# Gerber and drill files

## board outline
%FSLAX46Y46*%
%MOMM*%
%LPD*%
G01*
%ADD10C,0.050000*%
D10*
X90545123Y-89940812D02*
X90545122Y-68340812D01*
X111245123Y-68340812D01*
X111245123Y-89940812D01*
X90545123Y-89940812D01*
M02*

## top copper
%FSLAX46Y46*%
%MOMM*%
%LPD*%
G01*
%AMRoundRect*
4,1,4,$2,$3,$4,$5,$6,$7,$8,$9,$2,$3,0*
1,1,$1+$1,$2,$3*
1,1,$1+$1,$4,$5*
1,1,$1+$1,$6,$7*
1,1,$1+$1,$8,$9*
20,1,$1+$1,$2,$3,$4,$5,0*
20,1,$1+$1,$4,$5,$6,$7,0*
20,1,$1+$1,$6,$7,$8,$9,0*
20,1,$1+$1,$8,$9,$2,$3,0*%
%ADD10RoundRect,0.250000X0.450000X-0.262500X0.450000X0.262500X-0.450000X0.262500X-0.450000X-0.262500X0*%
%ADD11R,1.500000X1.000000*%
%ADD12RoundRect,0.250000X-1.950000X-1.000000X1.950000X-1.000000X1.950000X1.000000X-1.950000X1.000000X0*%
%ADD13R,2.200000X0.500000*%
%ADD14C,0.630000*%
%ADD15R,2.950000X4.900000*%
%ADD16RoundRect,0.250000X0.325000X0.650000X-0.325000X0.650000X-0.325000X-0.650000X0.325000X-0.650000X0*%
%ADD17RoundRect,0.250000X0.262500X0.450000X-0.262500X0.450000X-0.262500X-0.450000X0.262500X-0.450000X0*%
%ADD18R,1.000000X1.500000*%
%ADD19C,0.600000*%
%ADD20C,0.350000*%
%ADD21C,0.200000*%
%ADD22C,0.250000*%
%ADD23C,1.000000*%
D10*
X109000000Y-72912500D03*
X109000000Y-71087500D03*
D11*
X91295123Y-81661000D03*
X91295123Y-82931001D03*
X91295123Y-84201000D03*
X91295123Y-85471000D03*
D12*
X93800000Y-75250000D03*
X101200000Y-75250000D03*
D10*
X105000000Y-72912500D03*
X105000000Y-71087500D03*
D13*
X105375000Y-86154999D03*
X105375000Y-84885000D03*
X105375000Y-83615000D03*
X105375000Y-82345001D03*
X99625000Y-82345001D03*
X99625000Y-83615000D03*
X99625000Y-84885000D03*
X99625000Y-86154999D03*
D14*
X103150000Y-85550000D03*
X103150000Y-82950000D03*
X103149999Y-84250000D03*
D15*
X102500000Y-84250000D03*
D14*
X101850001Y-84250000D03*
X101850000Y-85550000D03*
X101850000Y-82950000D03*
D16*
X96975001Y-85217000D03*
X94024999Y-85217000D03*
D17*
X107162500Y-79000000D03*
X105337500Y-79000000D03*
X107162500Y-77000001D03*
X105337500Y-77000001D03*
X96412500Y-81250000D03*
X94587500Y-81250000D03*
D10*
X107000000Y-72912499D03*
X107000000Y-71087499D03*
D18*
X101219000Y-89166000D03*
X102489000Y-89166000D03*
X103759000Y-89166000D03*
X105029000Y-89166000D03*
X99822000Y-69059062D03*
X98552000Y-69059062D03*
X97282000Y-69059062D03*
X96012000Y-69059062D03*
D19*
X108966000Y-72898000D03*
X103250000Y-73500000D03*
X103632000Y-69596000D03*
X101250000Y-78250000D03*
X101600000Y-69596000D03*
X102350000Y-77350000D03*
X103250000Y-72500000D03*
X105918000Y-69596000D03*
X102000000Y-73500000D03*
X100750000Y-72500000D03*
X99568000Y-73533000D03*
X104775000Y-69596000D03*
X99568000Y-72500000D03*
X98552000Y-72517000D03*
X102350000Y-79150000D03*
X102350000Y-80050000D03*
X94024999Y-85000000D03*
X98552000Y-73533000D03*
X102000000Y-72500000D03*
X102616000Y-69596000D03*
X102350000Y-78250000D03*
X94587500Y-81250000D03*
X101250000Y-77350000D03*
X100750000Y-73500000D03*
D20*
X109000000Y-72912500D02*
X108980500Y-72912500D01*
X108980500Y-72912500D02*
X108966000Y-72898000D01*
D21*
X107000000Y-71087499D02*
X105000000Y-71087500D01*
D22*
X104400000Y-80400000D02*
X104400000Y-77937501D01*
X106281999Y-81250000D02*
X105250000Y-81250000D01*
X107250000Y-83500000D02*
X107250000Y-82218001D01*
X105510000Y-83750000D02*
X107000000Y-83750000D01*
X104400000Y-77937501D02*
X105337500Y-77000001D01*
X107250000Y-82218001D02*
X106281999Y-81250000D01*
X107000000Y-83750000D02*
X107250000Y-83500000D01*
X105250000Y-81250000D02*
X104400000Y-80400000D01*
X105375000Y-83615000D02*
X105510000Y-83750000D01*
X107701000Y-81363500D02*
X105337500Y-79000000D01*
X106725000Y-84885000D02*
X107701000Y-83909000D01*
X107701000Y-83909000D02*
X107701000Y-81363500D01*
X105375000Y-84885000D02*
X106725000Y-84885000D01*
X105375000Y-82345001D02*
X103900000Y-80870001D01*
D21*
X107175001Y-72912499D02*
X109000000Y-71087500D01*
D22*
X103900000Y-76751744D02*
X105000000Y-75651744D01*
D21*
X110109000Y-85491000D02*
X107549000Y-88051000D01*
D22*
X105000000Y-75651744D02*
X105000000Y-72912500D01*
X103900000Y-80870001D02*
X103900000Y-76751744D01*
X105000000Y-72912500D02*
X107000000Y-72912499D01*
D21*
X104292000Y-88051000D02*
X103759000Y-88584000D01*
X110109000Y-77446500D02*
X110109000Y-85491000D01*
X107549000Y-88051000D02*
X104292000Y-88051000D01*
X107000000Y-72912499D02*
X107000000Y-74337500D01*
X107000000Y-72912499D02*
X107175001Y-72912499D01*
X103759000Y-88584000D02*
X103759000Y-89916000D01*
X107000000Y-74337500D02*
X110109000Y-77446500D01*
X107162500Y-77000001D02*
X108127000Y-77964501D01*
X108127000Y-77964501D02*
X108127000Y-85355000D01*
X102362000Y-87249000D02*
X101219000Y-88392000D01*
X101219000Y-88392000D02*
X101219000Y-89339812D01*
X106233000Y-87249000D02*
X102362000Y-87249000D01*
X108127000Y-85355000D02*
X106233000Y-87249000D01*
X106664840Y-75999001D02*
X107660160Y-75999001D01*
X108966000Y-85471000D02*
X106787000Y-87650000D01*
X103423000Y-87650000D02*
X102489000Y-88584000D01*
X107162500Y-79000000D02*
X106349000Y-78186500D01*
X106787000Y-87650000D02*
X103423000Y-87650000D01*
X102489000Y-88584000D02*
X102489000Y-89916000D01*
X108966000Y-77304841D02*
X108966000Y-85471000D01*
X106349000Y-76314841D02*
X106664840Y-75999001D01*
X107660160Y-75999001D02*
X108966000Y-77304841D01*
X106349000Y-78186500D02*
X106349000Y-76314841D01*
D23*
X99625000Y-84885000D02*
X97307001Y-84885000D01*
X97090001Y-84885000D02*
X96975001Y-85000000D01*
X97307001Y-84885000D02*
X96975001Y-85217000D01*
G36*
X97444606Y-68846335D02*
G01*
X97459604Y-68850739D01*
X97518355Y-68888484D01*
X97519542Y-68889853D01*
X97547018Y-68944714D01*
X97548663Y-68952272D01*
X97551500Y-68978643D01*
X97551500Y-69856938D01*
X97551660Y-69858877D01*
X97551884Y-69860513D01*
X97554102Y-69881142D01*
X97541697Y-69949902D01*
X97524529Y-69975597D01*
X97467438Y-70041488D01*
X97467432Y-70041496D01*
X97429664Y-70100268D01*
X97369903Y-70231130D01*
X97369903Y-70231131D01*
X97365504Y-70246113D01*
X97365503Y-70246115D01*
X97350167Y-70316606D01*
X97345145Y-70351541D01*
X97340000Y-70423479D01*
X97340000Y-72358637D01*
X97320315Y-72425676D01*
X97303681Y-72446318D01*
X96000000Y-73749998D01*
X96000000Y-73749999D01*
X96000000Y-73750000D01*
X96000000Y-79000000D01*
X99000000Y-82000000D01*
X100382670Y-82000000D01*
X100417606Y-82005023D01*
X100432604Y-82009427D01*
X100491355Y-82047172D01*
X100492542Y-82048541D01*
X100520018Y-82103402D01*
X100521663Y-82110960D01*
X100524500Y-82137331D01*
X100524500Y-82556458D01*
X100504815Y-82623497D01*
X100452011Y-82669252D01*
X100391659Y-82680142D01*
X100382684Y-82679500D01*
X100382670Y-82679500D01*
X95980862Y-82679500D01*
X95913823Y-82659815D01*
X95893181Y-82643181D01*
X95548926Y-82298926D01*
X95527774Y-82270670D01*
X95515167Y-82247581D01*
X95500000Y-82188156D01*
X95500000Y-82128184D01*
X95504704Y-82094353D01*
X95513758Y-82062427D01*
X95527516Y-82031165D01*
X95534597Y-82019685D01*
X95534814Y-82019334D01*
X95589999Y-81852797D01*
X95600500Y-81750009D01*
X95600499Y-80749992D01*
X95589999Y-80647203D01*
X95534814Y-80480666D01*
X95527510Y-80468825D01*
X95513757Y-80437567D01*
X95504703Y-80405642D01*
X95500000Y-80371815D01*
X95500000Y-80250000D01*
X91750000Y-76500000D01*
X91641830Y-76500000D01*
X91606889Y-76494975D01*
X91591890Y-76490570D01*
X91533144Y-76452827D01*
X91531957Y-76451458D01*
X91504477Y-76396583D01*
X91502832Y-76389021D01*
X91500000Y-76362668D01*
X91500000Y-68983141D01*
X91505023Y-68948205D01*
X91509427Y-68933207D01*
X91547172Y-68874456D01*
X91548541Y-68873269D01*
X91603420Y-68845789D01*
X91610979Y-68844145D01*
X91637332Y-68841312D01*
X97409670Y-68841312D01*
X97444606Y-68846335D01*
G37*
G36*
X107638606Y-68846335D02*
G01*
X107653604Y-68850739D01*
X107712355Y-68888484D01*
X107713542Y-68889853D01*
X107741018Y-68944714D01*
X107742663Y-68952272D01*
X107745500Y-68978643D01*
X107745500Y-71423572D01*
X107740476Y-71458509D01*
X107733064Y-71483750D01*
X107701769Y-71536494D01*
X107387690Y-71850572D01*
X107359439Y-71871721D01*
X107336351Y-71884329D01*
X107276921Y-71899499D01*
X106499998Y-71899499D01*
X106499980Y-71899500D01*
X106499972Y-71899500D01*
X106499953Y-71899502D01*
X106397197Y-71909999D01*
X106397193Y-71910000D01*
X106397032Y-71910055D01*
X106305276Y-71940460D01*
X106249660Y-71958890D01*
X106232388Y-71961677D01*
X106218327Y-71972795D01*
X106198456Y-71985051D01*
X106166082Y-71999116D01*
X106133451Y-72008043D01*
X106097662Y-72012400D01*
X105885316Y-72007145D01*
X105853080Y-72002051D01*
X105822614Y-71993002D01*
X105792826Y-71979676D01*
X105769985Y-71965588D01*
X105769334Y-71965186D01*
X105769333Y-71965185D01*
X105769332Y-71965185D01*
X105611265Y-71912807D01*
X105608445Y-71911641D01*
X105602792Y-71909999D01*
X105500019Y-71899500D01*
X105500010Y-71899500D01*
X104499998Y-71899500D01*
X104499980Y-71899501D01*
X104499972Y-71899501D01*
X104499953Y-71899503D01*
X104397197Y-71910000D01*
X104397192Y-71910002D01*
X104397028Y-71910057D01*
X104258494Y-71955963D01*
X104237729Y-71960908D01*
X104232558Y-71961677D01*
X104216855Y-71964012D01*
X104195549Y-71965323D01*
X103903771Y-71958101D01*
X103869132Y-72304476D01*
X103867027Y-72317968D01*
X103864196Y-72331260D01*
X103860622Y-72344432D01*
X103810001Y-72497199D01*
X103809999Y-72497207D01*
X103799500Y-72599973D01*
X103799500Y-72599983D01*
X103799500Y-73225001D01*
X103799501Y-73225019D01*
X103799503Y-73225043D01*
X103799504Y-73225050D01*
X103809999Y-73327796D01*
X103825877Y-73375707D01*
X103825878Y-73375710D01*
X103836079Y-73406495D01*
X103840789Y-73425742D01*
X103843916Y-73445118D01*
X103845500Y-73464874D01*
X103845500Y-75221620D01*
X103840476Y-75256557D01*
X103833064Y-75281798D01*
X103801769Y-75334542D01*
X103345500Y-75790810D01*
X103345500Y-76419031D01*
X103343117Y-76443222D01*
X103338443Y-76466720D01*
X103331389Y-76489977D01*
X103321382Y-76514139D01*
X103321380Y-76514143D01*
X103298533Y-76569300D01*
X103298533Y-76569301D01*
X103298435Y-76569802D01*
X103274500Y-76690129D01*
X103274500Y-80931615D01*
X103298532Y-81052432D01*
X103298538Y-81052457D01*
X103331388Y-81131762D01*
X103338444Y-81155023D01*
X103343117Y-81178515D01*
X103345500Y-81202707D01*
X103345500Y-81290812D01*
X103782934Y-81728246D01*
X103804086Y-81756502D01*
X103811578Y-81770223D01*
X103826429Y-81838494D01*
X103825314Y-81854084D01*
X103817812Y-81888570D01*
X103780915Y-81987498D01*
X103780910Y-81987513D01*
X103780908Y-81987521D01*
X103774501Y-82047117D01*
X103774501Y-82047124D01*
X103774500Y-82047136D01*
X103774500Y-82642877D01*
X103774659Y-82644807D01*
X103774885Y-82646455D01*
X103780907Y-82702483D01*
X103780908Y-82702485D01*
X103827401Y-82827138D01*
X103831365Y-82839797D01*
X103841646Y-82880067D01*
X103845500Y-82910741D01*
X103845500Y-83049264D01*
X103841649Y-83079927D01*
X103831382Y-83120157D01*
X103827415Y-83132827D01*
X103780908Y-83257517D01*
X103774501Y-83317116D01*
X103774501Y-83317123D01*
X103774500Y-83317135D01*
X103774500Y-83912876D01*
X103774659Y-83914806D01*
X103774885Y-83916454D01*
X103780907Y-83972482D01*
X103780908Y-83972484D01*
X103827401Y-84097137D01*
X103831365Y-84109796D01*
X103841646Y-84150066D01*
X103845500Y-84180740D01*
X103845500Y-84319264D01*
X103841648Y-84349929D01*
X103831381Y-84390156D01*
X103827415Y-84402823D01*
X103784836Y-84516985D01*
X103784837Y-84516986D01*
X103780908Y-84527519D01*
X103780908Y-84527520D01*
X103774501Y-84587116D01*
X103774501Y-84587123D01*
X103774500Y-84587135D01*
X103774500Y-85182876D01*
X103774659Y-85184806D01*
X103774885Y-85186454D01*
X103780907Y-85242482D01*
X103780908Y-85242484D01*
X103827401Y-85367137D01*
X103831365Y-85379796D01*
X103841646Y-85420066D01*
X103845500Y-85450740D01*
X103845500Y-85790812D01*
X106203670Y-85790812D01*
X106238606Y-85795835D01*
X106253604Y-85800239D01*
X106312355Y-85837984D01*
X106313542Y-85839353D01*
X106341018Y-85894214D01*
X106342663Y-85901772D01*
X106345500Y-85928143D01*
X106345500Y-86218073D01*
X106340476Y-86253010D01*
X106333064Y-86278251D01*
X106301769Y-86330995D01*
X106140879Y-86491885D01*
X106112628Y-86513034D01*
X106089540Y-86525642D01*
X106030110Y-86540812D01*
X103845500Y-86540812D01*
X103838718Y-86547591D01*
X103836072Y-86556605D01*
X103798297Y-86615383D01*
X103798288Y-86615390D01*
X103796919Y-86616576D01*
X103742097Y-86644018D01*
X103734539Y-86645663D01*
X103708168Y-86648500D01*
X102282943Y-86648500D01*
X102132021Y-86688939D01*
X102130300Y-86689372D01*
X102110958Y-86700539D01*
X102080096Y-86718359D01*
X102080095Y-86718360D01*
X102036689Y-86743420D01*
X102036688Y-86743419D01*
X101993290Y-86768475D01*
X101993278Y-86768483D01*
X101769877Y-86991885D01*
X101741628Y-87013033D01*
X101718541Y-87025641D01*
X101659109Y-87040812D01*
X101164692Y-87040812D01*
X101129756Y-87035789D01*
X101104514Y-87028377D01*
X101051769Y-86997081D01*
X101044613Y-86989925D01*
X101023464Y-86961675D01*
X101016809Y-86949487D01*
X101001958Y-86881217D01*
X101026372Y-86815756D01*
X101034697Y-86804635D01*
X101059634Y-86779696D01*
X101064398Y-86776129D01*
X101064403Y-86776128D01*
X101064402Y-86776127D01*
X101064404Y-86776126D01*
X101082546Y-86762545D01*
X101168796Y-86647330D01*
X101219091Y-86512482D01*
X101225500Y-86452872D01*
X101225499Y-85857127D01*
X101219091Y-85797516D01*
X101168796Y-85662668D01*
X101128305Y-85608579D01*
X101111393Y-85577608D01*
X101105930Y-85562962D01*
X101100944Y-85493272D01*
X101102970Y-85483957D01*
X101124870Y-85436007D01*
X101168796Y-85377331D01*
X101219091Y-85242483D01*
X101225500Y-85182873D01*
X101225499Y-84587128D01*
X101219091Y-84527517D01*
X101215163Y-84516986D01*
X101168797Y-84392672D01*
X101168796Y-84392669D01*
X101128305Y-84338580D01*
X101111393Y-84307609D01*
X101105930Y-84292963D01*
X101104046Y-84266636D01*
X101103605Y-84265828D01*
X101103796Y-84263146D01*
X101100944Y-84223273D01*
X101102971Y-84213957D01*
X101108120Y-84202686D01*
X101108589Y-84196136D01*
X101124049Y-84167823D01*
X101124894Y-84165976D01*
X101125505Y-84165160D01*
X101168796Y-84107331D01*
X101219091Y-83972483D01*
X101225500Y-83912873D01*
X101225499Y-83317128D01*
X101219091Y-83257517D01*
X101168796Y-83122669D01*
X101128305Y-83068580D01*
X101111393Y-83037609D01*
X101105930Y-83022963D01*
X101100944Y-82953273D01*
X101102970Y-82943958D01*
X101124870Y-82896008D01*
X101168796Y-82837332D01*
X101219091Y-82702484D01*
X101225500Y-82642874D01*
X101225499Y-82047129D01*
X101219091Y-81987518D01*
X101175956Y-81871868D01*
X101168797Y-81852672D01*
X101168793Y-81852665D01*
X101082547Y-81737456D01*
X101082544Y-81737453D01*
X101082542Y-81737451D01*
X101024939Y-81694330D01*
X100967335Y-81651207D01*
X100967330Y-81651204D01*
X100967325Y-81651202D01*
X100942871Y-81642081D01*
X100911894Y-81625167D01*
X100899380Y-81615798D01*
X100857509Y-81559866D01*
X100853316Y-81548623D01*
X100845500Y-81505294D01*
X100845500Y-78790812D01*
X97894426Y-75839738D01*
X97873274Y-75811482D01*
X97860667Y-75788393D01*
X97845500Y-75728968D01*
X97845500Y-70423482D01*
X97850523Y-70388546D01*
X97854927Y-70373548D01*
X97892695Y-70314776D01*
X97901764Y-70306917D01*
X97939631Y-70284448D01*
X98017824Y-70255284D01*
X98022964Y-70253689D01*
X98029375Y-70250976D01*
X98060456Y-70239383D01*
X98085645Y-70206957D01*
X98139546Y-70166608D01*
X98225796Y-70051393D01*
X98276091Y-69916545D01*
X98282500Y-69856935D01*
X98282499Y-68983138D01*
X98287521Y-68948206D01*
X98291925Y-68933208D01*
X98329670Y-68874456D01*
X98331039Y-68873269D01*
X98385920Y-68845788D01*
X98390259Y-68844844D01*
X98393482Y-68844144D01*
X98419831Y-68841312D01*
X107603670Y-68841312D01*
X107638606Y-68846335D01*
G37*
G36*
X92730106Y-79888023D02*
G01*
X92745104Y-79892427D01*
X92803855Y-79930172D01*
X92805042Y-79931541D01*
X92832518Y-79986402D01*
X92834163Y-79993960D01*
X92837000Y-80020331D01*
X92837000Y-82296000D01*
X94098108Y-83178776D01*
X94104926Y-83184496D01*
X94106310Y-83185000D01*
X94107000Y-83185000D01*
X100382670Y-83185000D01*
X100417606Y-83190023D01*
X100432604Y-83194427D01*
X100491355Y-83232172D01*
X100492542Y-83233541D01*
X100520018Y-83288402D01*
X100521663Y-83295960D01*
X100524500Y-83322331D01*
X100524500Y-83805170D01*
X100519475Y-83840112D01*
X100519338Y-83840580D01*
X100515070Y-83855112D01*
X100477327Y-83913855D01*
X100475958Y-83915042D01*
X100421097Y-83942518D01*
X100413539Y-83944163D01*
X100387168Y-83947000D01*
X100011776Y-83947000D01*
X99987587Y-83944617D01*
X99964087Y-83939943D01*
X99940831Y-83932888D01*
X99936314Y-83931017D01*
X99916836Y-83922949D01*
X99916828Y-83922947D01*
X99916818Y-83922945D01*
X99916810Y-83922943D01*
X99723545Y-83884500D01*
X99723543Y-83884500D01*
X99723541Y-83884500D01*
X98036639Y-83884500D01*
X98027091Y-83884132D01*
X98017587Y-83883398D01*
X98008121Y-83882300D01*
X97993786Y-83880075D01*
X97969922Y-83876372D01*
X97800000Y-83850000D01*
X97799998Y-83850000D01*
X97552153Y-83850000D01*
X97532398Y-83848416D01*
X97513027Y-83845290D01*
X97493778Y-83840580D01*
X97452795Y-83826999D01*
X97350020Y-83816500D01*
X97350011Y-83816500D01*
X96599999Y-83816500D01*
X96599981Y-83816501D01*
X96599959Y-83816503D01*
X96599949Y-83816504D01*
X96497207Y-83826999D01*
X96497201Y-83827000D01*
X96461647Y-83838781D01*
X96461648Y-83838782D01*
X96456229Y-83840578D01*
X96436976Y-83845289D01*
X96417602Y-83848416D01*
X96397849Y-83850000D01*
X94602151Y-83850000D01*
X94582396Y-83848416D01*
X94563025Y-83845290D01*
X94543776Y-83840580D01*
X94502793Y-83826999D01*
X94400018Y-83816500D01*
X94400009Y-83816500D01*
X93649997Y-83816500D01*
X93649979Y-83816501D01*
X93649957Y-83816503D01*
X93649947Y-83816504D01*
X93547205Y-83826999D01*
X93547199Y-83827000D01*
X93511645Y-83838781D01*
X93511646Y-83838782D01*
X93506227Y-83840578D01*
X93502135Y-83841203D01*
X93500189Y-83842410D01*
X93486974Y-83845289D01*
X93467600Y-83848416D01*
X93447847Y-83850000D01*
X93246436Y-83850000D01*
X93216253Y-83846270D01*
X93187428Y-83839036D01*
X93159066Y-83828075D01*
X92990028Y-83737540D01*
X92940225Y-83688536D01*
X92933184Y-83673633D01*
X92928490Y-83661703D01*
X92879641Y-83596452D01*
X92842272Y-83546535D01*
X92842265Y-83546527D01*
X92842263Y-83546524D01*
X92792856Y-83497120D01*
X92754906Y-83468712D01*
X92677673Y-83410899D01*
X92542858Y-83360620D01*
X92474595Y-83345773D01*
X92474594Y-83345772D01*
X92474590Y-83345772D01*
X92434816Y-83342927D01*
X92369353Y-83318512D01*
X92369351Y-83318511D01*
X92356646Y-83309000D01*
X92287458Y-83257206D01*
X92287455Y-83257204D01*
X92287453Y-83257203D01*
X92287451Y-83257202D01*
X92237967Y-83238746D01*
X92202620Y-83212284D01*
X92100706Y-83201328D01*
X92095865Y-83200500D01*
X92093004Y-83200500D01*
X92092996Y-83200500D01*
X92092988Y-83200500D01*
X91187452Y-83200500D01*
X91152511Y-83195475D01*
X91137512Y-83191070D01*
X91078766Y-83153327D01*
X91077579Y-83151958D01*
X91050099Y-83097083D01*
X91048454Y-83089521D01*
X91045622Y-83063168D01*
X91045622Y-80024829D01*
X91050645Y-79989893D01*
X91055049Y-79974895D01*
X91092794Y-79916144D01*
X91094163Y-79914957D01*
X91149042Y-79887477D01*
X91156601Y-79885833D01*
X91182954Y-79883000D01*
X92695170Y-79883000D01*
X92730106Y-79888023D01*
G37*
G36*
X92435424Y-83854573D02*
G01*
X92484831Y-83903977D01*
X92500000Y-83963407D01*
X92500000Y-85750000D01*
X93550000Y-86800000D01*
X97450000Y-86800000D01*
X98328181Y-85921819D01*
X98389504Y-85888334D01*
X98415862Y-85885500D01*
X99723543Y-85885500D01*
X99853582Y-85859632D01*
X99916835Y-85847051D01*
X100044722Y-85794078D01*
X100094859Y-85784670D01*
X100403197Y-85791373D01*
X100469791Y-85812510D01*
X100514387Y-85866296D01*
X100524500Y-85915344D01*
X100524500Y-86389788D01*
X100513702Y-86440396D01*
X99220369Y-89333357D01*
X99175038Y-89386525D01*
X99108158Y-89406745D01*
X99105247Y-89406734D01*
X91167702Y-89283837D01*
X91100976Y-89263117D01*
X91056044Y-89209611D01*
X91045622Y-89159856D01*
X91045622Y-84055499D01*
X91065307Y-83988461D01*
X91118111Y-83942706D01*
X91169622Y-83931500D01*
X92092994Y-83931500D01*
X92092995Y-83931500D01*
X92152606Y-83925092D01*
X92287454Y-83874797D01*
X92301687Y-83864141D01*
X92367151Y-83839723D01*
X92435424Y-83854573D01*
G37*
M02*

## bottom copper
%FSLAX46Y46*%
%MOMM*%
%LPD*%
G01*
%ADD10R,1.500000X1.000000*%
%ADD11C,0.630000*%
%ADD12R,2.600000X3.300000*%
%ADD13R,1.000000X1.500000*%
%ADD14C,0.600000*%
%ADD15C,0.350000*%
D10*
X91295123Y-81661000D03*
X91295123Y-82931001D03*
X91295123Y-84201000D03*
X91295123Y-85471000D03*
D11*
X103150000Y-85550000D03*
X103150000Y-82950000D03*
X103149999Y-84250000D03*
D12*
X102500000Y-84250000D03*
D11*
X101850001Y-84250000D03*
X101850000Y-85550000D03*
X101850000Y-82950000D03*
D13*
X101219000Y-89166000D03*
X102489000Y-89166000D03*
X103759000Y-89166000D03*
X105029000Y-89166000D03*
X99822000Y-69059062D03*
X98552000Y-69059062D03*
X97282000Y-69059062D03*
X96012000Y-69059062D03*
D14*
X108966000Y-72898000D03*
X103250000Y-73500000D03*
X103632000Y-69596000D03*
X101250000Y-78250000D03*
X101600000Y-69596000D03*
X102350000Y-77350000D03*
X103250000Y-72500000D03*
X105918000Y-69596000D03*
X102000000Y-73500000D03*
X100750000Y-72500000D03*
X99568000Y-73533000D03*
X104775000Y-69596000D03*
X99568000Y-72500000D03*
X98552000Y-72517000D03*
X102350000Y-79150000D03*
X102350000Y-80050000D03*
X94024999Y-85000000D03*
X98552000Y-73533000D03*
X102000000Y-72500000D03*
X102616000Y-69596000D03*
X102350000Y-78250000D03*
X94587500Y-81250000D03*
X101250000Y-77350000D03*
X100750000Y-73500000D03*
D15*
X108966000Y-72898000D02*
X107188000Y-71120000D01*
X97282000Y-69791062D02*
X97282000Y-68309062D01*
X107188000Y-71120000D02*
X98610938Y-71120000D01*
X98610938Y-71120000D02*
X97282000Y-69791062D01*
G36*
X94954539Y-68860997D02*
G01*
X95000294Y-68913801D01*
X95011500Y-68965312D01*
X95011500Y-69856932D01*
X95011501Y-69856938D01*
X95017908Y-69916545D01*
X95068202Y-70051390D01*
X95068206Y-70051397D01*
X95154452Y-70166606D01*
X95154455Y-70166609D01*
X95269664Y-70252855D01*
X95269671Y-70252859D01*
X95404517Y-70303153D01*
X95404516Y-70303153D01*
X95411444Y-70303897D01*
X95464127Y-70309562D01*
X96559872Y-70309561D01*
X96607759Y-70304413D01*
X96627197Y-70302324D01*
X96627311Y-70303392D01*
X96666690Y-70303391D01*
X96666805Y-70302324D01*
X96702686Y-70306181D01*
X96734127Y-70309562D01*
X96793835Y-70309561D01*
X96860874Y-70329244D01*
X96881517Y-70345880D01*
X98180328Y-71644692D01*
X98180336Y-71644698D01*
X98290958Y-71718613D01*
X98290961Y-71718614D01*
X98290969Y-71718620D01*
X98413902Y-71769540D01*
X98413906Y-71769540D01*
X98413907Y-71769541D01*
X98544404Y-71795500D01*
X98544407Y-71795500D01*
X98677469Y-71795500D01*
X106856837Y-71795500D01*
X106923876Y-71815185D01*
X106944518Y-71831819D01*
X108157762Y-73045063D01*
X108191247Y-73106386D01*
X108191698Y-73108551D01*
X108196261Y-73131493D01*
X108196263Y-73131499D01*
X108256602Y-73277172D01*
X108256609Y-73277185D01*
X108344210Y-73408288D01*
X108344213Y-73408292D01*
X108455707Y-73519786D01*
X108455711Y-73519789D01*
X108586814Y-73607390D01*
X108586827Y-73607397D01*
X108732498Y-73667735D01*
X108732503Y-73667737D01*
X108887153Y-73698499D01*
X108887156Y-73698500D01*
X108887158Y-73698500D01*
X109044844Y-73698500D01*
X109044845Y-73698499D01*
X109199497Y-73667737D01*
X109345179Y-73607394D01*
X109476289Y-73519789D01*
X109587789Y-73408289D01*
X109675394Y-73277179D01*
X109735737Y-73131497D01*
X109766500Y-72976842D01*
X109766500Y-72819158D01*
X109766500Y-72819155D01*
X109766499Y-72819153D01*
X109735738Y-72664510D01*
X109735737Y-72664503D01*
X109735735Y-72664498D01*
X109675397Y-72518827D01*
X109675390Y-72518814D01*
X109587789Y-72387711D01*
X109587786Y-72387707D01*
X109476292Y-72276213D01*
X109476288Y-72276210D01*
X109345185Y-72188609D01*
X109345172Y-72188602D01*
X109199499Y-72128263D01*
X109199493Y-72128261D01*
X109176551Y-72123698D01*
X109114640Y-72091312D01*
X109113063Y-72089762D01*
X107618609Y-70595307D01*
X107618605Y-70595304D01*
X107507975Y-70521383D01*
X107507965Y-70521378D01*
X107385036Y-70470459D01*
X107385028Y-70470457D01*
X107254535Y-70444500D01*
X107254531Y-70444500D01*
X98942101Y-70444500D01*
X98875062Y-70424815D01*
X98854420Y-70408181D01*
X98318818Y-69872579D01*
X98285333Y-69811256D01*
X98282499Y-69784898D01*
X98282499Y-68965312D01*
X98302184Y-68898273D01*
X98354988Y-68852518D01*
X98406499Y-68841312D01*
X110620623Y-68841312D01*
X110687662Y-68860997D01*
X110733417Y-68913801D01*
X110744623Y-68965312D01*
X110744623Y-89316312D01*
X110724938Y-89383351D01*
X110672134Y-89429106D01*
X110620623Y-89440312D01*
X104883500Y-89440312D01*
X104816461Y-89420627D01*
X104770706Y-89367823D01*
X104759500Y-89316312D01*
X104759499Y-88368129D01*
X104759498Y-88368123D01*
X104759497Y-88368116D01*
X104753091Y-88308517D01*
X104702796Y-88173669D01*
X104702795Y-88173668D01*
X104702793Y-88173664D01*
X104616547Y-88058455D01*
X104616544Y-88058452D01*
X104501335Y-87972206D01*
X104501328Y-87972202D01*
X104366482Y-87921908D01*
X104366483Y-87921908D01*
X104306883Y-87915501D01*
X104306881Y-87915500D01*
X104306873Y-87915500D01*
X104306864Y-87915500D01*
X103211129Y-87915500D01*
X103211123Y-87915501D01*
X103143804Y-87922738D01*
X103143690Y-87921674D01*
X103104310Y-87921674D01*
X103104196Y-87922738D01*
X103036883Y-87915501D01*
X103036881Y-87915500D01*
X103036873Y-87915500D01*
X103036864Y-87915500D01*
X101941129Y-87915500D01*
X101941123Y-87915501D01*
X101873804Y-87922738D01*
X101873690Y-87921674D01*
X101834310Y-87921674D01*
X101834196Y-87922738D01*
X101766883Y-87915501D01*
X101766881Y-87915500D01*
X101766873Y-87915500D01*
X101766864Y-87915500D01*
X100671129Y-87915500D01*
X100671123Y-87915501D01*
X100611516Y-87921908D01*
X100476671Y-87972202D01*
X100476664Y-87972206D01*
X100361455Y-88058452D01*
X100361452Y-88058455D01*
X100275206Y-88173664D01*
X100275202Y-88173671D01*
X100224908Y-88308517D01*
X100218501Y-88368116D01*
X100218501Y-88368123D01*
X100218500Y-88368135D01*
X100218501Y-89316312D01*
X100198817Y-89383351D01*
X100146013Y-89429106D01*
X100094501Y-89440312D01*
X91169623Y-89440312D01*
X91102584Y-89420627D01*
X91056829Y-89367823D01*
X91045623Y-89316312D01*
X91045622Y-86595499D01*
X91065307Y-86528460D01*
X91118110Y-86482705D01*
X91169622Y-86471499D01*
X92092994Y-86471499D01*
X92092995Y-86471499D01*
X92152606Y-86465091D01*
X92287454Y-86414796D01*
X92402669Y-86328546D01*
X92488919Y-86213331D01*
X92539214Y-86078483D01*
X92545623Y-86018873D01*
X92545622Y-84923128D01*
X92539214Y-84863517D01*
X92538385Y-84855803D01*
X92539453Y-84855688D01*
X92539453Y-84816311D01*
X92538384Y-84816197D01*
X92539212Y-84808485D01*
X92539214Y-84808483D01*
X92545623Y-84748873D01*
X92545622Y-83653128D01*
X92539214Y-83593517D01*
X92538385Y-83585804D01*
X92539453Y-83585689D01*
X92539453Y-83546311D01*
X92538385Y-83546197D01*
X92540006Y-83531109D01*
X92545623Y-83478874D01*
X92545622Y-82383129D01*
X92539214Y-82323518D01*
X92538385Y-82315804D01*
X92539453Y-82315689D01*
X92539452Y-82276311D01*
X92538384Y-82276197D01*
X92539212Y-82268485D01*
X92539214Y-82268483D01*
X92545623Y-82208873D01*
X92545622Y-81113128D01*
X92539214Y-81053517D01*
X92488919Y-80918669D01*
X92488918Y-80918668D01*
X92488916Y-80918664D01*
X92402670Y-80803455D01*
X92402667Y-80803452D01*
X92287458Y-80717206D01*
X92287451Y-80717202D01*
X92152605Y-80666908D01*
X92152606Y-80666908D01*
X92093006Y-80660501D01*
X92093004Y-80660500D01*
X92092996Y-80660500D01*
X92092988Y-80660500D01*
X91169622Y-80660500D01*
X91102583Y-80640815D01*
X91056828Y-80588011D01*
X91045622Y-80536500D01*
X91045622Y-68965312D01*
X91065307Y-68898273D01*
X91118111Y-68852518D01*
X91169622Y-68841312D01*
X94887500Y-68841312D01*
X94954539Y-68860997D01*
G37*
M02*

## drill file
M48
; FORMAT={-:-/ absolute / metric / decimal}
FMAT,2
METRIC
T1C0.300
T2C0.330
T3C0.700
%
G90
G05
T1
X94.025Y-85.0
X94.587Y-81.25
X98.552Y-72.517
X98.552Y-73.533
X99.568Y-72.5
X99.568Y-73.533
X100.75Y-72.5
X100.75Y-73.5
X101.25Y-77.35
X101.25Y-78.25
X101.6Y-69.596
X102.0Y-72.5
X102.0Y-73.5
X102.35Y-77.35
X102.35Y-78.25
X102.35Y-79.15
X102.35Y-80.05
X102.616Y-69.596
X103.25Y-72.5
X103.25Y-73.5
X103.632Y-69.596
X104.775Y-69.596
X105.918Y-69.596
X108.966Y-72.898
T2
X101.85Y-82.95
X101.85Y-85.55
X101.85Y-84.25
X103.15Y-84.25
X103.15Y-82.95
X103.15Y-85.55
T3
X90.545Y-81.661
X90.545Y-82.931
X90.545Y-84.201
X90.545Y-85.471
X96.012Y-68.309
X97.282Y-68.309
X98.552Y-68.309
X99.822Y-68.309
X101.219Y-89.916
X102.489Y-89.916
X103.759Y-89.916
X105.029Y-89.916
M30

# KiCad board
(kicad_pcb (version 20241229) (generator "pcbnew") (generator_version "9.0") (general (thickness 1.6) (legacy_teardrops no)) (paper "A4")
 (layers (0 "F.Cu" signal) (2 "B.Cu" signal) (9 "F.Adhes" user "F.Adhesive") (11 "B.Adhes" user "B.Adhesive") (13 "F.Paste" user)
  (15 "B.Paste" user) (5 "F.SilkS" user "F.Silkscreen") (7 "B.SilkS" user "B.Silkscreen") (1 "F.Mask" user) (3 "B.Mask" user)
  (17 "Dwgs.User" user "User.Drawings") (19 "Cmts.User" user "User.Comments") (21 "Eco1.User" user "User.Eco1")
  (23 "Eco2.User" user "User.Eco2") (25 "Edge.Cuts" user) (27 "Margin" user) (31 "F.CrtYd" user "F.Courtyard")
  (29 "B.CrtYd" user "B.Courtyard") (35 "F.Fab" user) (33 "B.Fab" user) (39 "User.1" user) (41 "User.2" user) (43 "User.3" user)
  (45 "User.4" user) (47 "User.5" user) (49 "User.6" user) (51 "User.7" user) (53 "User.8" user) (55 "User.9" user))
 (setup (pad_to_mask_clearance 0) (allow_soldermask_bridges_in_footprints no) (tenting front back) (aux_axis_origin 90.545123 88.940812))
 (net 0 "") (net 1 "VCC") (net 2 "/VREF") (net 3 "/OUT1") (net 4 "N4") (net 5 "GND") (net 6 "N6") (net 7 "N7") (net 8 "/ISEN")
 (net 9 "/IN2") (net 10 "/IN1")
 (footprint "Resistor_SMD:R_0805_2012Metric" (layer "F.Cu") (at 109 72 90)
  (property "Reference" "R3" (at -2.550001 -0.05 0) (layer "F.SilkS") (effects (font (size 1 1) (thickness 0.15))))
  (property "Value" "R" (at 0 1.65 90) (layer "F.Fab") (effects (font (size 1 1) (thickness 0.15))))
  (pad "1" smd roundrect (at -0.9125 0 90) (size 1.025 1.4) (layers "F.Cu" "F.Mask" "F.Paste") (roundrect_rratio 0.243902) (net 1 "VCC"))
  (pad "2" smd roundrect (at 0.9125 0 90) (size 1.025 1.4) (layers "F.Cu" "F.Mask" "F.Paste") (roundrect_rratio 0.243902) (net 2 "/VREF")))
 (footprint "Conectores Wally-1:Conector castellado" (layer "F.Cu") (at 90.682623 83.3835 180)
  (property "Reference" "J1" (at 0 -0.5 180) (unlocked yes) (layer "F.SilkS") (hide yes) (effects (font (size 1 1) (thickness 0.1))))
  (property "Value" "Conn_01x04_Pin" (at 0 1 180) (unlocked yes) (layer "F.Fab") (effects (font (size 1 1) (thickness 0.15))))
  (pad "1" thru_hole rect (at 0.1375 1.7225) (size 1.5 1) (drill 0.7 (offset 0.75 0)) (layers "*.Cu" "*.Mask") (remove_unused_layers no)
   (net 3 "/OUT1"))
  (pad "2" thru_hole rect (at 0.1375 0.452499) (size 1.5 1) (drill 0.7 (offset 0.75 0)) (layers "*.Cu" "*.Mask") (remove_unused_layers no)
   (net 3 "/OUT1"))
  (pad "3" thru_hole rect (at 0.1375 -0.8175) (size 1.5 1) (drill 0.7 (offset 0.75 0)) (layers "*.Cu" "*.Mask") (remove_unused_layers no)
   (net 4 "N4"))
  (pad "4" thru_hole rect (at 0.1375 -2.0875) (size 1.5 1) (drill 0.7 (offset 0.75 0)) (layers "*.Cu" "*.Mask") (remove_unused_layers no)
   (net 4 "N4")))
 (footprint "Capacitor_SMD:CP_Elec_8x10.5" (layer "F.Cu") (at 97.5 75.25)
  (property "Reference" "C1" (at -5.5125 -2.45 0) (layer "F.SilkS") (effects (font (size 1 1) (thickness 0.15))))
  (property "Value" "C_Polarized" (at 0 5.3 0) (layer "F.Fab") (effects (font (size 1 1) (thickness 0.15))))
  (pad "1" smd roundrect (at -3.7 0) (size 4.4 2.5) (layers "F.Cu" "F.Mask" "F.Paste") (roundrect_rratio 0.1) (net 1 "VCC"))
  (pad "2" smd roundrect (at 3.7 0) (size 4.4 2.5) (layers "F.Cu" "F.Mask" "F.Paste") (roundrect_rratio 0.1) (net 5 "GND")))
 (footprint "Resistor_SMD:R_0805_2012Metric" (layer "F.Cu") (at 105 72 90)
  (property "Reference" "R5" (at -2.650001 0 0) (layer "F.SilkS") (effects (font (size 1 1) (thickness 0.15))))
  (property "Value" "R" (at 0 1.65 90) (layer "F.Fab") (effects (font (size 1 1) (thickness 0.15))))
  (pad "1" smd roundrect (at -0.9125 0 90) (size 1.025 1.4) (layers "F.Cu" "F.Mask" "F.Paste") (roundrect_rratio 0.243902) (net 2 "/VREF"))
  (pad "2" smd roundrect (at 0.9125 0 90) (size 1.025 1.4) (layers "F.Cu" "F.Mask" "F.Paste") (roundrect_rratio 0.243902) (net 5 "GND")))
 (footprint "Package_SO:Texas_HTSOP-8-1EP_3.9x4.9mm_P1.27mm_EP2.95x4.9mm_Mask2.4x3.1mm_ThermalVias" (layer "F.Cu") (at 102.5 84.25 180)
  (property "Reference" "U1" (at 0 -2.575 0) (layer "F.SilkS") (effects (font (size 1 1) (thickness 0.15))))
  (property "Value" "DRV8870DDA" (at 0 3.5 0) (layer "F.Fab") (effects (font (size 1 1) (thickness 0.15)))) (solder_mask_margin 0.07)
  (pad "" smd rect (at 0 0 180) (size 2.4 3.1) (layers "F.Mask"))
  (pad "" smd rect (at 0 0 180) (size 2.4 3.1) (layers "F.Paste"))
  (pad "1" smd rect (at -2.875 -1.904999 180) (size 2.2 0.5) (layers "F.Cu" "F.Mask" "F.Paste") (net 5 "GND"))
  (pad "2" smd rect (at -2.875 -0.635 180) (size 2.2 0.5) (layers "F.Cu" "F.Mask" "F.Paste") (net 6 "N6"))
  (pad "3" smd rect (at -2.875 0.635 180) (size 2.2 0.5) (layers "F.Cu" "F.Mask" "F.Paste") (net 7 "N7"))
  (pad "4" smd rect (at -2.875 1.904999 180) (size 2.2 0.5) (layers "F.Cu" "F.Mask" "F.Paste") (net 2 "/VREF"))
  (pad "5" smd rect (at 2.875 1.904999 180) (size 2.2 0.5) (layers "F.Cu" "F.Mask" "F.Paste") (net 1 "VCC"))
  (pad "6" smd rect (at 2.875 0.635 180) (size 2.2 0.5) (layers "F.Cu" "F.Mask" "F.Paste") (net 3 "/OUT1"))
  (pad "7" smd rect (at 2.875 -0.635 180) (size 2.2 0.5) (layers "F.Cu" "F.Mask" "F.Paste") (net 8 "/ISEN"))
  (pad "8" smd rect (at 2.875 -1.904999 180) (size 2.2 0.5) (layers "F.Cu" "F.Mask" "F.Paste") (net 4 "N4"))
  (pad "9" thru_hole circle (at -0.65 -1.3 180) (size 0.63 0.63) (drill 0.33) (layers "*.Cu" "*.Mask") (remove_unused_layers no)
   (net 5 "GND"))
  (pad "9" thru_hole circle (at -0.65 1.3 180) (size 0.63 0.63) (drill 0.33) (layers "*.Cu" "*.Mask") (remove_unused_layers no)
   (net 5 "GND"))
  (pad "9" thru_hole circle (at -0.649999 0 180) (size 0.63 0.63) (drill 0.33) (layers "*.Cu" "*.Mask") (remove_unused_layers no)
   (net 5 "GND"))
  (pad "9" smd rect (at 0 0 180) (size 2.6 3.3) (layers "B.Cu") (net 5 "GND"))
  (pad "9" smd rect (at 0 0 180) (size 2.95 4.9) (layers "F.Cu") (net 5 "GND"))
  (pad "9" thru_hole circle (at 0.649999 0 180) (size 0.63 0.63) (drill 0.33) (layers "*.Cu" "*.Mask") (remove_unused_layers no)
   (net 5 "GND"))
  (pad "9" thru_hole circle (at 0.65 -1.3 180) (size 0.63 0.63) (drill 0.33) (layers "*.Cu" "*.Mask") (remove_unused_layers no)
   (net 5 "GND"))
  (pad "9" thru_hole circle (at 0.65 1.3 180) (size 0.63 0.63) (drill 0.33) (layers "*.Cu" "*.Mask") (remove_unused_layers no) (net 5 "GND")))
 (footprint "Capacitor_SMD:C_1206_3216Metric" (layer "F.Cu") (at 95.5 85.217 180)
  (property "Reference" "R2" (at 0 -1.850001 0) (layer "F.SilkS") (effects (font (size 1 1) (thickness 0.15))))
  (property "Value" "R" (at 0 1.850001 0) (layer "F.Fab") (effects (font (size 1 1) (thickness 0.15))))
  (pad "1" smd roundrect (at -1.475001 0 180) (size 1.15 1.8) (layers "F.Cu" "F.Mask" "F.Paste") (roundrect_rratio 0.217391) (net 8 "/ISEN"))
  (pad "2" smd roundrect (at 1.475001 0 180) (size 1.15 1.8) (layers "F.Cu" "F.Mask" "F.Paste") (roundrect_rratio 0.217391) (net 5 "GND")))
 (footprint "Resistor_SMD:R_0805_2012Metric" (layer "F.Cu") (at 106.25 79 180)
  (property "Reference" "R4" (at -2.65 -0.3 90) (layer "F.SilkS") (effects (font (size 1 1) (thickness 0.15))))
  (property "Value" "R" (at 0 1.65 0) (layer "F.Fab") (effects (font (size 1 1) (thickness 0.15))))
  (pad "1" smd roundrect (at -0.9125 0 180) (size 1.025 1.4) (layers "F.Cu" "F.Mask" "F.Paste") (roundrect_rratio 0.243902) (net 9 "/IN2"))
  (pad "2" smd roundrect (at 0.9125 0 180) (size 1.025 1.4) (layers "F.Cu" "F.Mask" "F.Paste") (roundrect_rratio 0.243902) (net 6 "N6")))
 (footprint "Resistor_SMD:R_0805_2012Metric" (layer "F.Cu") (at 106.25 77.000001 180)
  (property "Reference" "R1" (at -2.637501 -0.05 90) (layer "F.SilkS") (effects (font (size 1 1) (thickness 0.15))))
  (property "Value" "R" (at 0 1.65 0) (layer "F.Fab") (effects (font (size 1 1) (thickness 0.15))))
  (pad "1" smd roundrect (at -0.9125 0 180) (size 1.025 1.4) (layers "F.Cu" "F.Mask" "F.Paste") (roundrect_rratio 0.243902) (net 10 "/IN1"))
  (pad "2" smd roundrect (at 0.9125 0 180) (size 1.025 1.4) (layers "F.Cu" "F.Mask" "F.Paste") (roundrect_rratio 0.243902) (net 7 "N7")))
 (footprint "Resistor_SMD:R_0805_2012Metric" (layer "F.Cu") (at 95.5 81.25 180)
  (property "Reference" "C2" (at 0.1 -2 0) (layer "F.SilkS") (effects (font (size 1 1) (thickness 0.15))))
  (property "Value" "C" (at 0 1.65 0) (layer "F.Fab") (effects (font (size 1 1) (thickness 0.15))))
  (pad "1" smd roundrect (at -0.9125 0 180) (size 1.025 1.4) (layers "F.Cu" "F.Mask" "F.Paste") (roundrect_rratio 0.243902) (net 1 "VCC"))
  (pad "2" smd roundrect (at 0.9125 0 180) (size 1.025 1.4) (layers "F.Cu" "F.Mask" "F.Paste") (roundrect_rratio 0.243902) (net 5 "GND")))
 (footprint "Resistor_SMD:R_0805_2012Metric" (layer "F.Cu") (at 107 71.999999 90)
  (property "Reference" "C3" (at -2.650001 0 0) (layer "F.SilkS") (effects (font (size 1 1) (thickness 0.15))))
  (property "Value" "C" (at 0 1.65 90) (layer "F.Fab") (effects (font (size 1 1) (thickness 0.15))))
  (pad "1" smd roundrect (at -0.9125 0 90) (size 1.025 1.4) (layers "F.Cu" "F.Mask" "F.Paste") (roundrect_rratio 0.243902) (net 2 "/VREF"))
  (pad "2" smd roundrect (at 0.9125 0 90) (size 1.025 1.4) (layers "F.Cu" "F.Mask" "F.Paste") (roundrect_rratio 0.243902) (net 5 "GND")))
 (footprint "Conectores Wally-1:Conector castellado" (layer "F.Cu") (at 102.9415 89.7785 -90)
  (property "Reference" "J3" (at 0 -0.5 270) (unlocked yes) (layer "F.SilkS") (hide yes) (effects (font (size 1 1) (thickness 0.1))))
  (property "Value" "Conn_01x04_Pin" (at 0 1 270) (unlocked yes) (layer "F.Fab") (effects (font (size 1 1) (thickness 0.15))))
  (pad "1" thru_hole rect (at 0.1375 1.7225 90) (size 1.5 1) (drill 0.7 (offset 0.75 0)) (layers "*.Cu" "*.Mask") (remove_unused_layers no)
   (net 10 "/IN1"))
  (pad "2" thru_hole rect (at 0.1375 0.4525 90) (size 1.5 1) (drill 0.7 (offset 0.75 0)) (layers "*.Cu" "*.Mask") (remove_unused_layers no)
   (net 9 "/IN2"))
  (pad "3" thru_hole rect (at 0.1375 -0.8175 90) (size 1.5 1) (drill 0.7 (offset 0.75 0)) (layers "*.Cu" "*.Mask") (remove_unused_layers no)
   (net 2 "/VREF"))
  (pad "4" thru_hole rect (at 0.1375 -2.0875 90) (size 1.5 1) (drill 0.7 (offset 0.75 0)) (layers "*.Cu" "*.Mask") (remove_unused_layers no)
   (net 5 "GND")))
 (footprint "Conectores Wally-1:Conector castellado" (layer "F.Cu") (at 98.0995 68.446562 90)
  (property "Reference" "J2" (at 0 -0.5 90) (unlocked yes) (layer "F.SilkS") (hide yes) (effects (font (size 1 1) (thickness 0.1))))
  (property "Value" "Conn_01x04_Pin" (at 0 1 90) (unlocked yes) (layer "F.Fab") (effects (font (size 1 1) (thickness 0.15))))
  (pad "1" thru_hole rect (at 0.1375 1.7225 270) (size 1.5 1) (drill 0.7 (offset 0.75 0)) (layers "*.Cu" "*.Mask") (remove_unused_layers no)
   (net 5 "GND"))
  (pad "2" thru_hole rect (at 0.1375 0.4525 270) (size 1.5 1) (drill 0.7 (offset 0.75 0)) (layers "*.Cu" "*.Mask") (remove_unused_layers no)
   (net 5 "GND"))
  (pad "3" thru_hole rect (at 0.1375 -0.8175 270) (size 1.5 1) (drill 0.7 (offset 0.75 0)) (layers "*.Cu" "*.Mask")
   (remove_unused_layers no) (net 1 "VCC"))
  (pad "4" thru_hole rect (at 0.1375 -2.0875 270) (size 1.5 1) (drill 0.7 (offset 0.75 0)) (layers "*.Cu" "*.Mask")
   (remove_unused_layers no) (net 1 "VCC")))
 (gr_poly
  (pts (xy 90.545123 89.940812) (xy 90.545122 68.340812) (xy 111.245123 68.340812) (xy 111.245123 89.940812))
  (stroke (width 0.05) (type default)) (fill no) (layer "Edge.Cuts"))
 (segment (start 109 72.9125) (end 108.9805 72.9125) (width 0.35) (layer "F.Cu") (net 1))
 (segment (start 108.9805 72.9125) (end 108.966 72.898) (width 0.35) (layer "F.Cu") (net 1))
 (via (at 108.966 72.898) (size 0.6) (drill 0.3) (layers "F.Cu" "B.Cu") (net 1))
 (segment (start 108.966 72.898) (end 107.188 71.12) (width 0.35) (layer "B.Cu") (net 1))
 (segment (start 97.282 69.791062) (end 97.282 68.309062) (width 0.35) (layer "B.Cu") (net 1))
 (segment (start 107.188 71.12) (end 98.610938 71.12) (width 0.35) (layer "B.Cu") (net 1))
 (segment (start 98.610938 71.12) (end 97.282 69.791062) (width 0.35) (layer "B.Cu") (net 1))
 (segment (start 107 71.087499) (end 105 71.0875) (width 0.2) (layer "F.Cu") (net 5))
 (via (at 103.25 73.5) (size 0.6) (drill 0.3) (layers "F.Cu" "B.Cu") (free yes) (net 5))
 (via (at 103.632 69.596) (size 0.6) (drill 0.3) (layers "F.Cu" "B.Cu") (free yes) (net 5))
 (via (at 101.25 78.25) (size 0.6) (drill 0.3) (layers "F.Cu" "B.Cu") (free yes) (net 5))
 (via (at 101.6 69.596) (size 0.6) (drill 0.3) (layers "F.Cu" "B.Cu") (free yes) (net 5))
 (via (at 102.35 77.35) (size 0.6) (drill 0.3) (layers "F.Cu" "B.Cu") (free yes) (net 5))
 (via (at 103.25 72.5) (size 0.6) (drill 0.3) (layers "F.Cu" "B.Cu") (free yes) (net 5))
 (via (at 105.918 69.596) (size 0.6) (drill 0.3) (layers "F.Cu" "B.Cu") (free yes) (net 5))
 (via (at 102 73.5) (size 0.6) (drill 0.3) (layers "F.Cu" "B.Cu") (free yes) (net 5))
 (via (at 100.75 72.5) (size 0.6) (drill 0.3) (layers "F.Cu" "B.Cu") (free yes) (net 5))
 (via (at 99.568 73.533) (size 0.6) (drill 0.3) (layers "F.Cu" "B.Cu") (free yes) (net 5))
 (via (at 104.775 69.596) (size 0.6) (drill 0.3) (layers "F.Cu" "B.Cu") (free yes) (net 5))
 (via (at 99.568 72.5) (size 0.6) (drill 0.3) (layers "F.Cu" "B.Cu") (free yes) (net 5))
 (via (at 98.552 72.517) (size 0.6) (drill 0.3) (layers "F.Cu" "B.Cu") (free yes) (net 5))
 (via (at 102.35 79.15) (size 0.6) (drill 0.3) (layers "F.Cu" "B.Cu") (free yes) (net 5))
 (via (at 102.35 80.05) (size 0.6) (drill 0.3) (layers "F.Cu" "B.Cu") (free yes) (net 5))
 (via (at 94.024999 85) (size 0.6) (drill 0.3) (layers "F.Cu" "B.Cu") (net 5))
 (via (at 98.552 73.533) (size 0.6) (drill 0.3) (layers "F.Cu" "B.Cu") (free yes) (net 5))
 (via (at 102 72.5) (size 0.6) (drill 0.3) (layers "F.Cu" "B.Cu") (free yes) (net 5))
 (via (at 102.616 69.596) (size 0.6) (drill 0.3) (layers "F.Cu" "B.Cu") (free yes) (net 5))
 (via (at 102.35 78.25) (size 0.6) (drill 0.3) (layers "F.Cu" "B.Cu") (free yes) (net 5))
 (via (at 94.5875 81.25) (size 0.6) (drill 0.3) (layers "F.Cu" "B.Cu") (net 5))
 (via (at 101.25 77.35) (size 0.6) (drill 0.3) (layers "F.Cu" "B.Cu") (free yes) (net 5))
 (via (at 100.75 73.5) (size 0.6) (drill 0.3) (layers "F.Cu" "B.Cu") (free yes) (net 5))
 (segment (start 104.4 80.4) (end 104.4 77.937501) (width 0.25) (layer "F.Cu") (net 7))
 (segment (start 106.281999 81.25) (end 105.25 81.25) (width 0.25) (layer "F.Cu") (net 7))
 (segment (start 107.25 83.5) (end 107.25 82.218001) (width 0.25) (layer "F.Cu") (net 7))
 (segment (start 105.51 83.75) (end 107 83.75) (width 0.25) (layer "F.Cu") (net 7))
 (segment (start 104.4 77.937501) (end 105.3375 77.000001) (width 0.25) (layer "F.Cu") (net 7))
 (segment (start 107.25 82.218001) (end 106.281999 81.25) (width 0.25) (layer "F.Cu") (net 7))
 (segment (start 107 83.75) (end 107.25 83.5) (width 0.25) (layer "F.Cu") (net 7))
 (segment (start 105.25 81.25) (end 104.4 80.4) (width 0.25) (layer "F.Cu") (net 7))
 (segment (start 105.375 83.615) (end 105.51 83.75) (width 0.25) (layer "F.Cu") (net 7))
 (segment (start 107.701 81.3635) (end 105.3375 79) (width 0.25) (layer "F.Cu") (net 6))
 (segment (start 106.725 84.885) (end 107.701 83.909) (width 0.25) (layer "F.Cu") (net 6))
 (segment (start 107.701 83.909) (end 107.701 81.3635) (width 0.25) (layer "F.Cu") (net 6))
 (segment (start 105.375 84.885) (end 106.725 84.885) (width 0.25) (layer "F.Cu") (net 6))
 (segment (start 105.375 82.345001) (end 103.9 80.870001) (width 0.25) (layer "F.Cu") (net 2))
 (segment (start 107.175001 72.912499) (end 109 71.0875) (width 0.2) (layer "F.Cu") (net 2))
 (segment (start 103.9 76.751744) (end 105 75.651744) (width 0.25) (layer "F.Cu") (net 2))
 (segment (start 110.109 85.491) (end 107.549 88.051) (width 0.2) (layer "F.Cu") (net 2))
 (segment (start 105 75.651744) (end 105 72.9125) (width 0.25) (layer "F.Cu") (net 2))
 (segment (start 103.9 80.870001) (end 103.9 76.751744) (width 0.25) (layer "F.Cu") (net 2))
 (segment (start 105 72.9125) (end 107 72.912499) (width 0.25) (layer "F.Cu") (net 2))
 (segment (start 104.292 88.051) (end 103.759 88.584) (width 0.2) (layer "F.Cu") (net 2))
 (segment (start 110.109 77.4465) (end 110.109 85.491) (width 0.2) (layer "F.Cu") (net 2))
 (segment (start 107.549 88.051) (end 104.292 88.051) (width 0.2) (layer "F.Cu") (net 2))
 (segment (start 107 72.912499) (end 107 74.3375) (width 0.2) (layer "F.Cu") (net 2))
 (segment (start 107 72.912499) (end 107.175001 72.912499) (width 0.2) (layer "F.Cu") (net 2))
 (segment (start 103.759 88.584) (end 103.759 89.916) (width 0.2) (layer "F.Cu") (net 2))
 (segment (start 107 74.3375) (end 110.109 77.4465) (width 0.2) (layer "F.Cu") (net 2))
 (segment (start 107.1625 77.000001) (end 108.127 77.964501) (width 0.2) (layer "F.Cu") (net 10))
 (segment (start 108.127 77.964501) (end 108.127 85.355) (width 0.2) (layer "F.Cu") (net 10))
 (segment (start 102.362 87.249) (end 101.219 88.392) (width 0.2) (layer "F.Cu") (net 10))
 (segment (start 101.219 88.392) (end 101.219 89.339812) (width 0.2) (layer "F.Cu") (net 10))
 (segment (start 106.233 87.249) (end 102.362 87.249) (width 0.2) (layer "F.Cu") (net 10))
 (segment (start 108.127 85.355) (end 106.233 87.249) (width 0.2) (layer "F.Cu") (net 10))
 (segment (start 106.66484 75.999001) (end 107.66016 75.999001) (width 0.2) (layer "F.Cu") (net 9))
 (segment (start 108.966 85.471) (end 106.787 87.65) (width 0.2) (layer "F.Cu") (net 9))
 (segment (start 103.423 87.65) (end 102.489 88.584) (width 0.2) (layer "F.Cu") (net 9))
 (segment (start 107.1625 79) (end 106.349 78.1865) (width 0.2) (layer "F.Cu") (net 9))
 (segment (start 106.787 87.65) (end 103.423 87.65) (width 0.2) (layer "F.Cu") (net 9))
 (segment (start 102.489 88.584) (end 102.489 89.916) (width 0.2) (layer "F.Cu") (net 9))
 (segment (start 108.966 77.304841) (end 108.966 85.471) (width 0.2) (layer "F.Cu") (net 9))
 (segment (start 106.349 76.314841) (end 106.66484 75.999001) (width 0.2) (layer "F.Cu") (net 9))
 (segment (start 107.66016 75.999001) (end 108.966 77.304841) (width 0.2) (layer "F.Cu") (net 9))
 (segment (start 106.349 78.1865) (end 106.349 76.314841) (width 0.2) (layer "F.Cu") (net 9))
 (segment (start 99.625 84.885) (end 97.307001 84.885) (width 1) (layer "F.Cu") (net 8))
 (segment (start 97.090001 84.885) (end 96.975001 85) (width 1) (layer "F.Cu") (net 8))
 (segment (start 97.307001 84.885) (end 96.975001 85.217) (width 1) (layer "F.Cu") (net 8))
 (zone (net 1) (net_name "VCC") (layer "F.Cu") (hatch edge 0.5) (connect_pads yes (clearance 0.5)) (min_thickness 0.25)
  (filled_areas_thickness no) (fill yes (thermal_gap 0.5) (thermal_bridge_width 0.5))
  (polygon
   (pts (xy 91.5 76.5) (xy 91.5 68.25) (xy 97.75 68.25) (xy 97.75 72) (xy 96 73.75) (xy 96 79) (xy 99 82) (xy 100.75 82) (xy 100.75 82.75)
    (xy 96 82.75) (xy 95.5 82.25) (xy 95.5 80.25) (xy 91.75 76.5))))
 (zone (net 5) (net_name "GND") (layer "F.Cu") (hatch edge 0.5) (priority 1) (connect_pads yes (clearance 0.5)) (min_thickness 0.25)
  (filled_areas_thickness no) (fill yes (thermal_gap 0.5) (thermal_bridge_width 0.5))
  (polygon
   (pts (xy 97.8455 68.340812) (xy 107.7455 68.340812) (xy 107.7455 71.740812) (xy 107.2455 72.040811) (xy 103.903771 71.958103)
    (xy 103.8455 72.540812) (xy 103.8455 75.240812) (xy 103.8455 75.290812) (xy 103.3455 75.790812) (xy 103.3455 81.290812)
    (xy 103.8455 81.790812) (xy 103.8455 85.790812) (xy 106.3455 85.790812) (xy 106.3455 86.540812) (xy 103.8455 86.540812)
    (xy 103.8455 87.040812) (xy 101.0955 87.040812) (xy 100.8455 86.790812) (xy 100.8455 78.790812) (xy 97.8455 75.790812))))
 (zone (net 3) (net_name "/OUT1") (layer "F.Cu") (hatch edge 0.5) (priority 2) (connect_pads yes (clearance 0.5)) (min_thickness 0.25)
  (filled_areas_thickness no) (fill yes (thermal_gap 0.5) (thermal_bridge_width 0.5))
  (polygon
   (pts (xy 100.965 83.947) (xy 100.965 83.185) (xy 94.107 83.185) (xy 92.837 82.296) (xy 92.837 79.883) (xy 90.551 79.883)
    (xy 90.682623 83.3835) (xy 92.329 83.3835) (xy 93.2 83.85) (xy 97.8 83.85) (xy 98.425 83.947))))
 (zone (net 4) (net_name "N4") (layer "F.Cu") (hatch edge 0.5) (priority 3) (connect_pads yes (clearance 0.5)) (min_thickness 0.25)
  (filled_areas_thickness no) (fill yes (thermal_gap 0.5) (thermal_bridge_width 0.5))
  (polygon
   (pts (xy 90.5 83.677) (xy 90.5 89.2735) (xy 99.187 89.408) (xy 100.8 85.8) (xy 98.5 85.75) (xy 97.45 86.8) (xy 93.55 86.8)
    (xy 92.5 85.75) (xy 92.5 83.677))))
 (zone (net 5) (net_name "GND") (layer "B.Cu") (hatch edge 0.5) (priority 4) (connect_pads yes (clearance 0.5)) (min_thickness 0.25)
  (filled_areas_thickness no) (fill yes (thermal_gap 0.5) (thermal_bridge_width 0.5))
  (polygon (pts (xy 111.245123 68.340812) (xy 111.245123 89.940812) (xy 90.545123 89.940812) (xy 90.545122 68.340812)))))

